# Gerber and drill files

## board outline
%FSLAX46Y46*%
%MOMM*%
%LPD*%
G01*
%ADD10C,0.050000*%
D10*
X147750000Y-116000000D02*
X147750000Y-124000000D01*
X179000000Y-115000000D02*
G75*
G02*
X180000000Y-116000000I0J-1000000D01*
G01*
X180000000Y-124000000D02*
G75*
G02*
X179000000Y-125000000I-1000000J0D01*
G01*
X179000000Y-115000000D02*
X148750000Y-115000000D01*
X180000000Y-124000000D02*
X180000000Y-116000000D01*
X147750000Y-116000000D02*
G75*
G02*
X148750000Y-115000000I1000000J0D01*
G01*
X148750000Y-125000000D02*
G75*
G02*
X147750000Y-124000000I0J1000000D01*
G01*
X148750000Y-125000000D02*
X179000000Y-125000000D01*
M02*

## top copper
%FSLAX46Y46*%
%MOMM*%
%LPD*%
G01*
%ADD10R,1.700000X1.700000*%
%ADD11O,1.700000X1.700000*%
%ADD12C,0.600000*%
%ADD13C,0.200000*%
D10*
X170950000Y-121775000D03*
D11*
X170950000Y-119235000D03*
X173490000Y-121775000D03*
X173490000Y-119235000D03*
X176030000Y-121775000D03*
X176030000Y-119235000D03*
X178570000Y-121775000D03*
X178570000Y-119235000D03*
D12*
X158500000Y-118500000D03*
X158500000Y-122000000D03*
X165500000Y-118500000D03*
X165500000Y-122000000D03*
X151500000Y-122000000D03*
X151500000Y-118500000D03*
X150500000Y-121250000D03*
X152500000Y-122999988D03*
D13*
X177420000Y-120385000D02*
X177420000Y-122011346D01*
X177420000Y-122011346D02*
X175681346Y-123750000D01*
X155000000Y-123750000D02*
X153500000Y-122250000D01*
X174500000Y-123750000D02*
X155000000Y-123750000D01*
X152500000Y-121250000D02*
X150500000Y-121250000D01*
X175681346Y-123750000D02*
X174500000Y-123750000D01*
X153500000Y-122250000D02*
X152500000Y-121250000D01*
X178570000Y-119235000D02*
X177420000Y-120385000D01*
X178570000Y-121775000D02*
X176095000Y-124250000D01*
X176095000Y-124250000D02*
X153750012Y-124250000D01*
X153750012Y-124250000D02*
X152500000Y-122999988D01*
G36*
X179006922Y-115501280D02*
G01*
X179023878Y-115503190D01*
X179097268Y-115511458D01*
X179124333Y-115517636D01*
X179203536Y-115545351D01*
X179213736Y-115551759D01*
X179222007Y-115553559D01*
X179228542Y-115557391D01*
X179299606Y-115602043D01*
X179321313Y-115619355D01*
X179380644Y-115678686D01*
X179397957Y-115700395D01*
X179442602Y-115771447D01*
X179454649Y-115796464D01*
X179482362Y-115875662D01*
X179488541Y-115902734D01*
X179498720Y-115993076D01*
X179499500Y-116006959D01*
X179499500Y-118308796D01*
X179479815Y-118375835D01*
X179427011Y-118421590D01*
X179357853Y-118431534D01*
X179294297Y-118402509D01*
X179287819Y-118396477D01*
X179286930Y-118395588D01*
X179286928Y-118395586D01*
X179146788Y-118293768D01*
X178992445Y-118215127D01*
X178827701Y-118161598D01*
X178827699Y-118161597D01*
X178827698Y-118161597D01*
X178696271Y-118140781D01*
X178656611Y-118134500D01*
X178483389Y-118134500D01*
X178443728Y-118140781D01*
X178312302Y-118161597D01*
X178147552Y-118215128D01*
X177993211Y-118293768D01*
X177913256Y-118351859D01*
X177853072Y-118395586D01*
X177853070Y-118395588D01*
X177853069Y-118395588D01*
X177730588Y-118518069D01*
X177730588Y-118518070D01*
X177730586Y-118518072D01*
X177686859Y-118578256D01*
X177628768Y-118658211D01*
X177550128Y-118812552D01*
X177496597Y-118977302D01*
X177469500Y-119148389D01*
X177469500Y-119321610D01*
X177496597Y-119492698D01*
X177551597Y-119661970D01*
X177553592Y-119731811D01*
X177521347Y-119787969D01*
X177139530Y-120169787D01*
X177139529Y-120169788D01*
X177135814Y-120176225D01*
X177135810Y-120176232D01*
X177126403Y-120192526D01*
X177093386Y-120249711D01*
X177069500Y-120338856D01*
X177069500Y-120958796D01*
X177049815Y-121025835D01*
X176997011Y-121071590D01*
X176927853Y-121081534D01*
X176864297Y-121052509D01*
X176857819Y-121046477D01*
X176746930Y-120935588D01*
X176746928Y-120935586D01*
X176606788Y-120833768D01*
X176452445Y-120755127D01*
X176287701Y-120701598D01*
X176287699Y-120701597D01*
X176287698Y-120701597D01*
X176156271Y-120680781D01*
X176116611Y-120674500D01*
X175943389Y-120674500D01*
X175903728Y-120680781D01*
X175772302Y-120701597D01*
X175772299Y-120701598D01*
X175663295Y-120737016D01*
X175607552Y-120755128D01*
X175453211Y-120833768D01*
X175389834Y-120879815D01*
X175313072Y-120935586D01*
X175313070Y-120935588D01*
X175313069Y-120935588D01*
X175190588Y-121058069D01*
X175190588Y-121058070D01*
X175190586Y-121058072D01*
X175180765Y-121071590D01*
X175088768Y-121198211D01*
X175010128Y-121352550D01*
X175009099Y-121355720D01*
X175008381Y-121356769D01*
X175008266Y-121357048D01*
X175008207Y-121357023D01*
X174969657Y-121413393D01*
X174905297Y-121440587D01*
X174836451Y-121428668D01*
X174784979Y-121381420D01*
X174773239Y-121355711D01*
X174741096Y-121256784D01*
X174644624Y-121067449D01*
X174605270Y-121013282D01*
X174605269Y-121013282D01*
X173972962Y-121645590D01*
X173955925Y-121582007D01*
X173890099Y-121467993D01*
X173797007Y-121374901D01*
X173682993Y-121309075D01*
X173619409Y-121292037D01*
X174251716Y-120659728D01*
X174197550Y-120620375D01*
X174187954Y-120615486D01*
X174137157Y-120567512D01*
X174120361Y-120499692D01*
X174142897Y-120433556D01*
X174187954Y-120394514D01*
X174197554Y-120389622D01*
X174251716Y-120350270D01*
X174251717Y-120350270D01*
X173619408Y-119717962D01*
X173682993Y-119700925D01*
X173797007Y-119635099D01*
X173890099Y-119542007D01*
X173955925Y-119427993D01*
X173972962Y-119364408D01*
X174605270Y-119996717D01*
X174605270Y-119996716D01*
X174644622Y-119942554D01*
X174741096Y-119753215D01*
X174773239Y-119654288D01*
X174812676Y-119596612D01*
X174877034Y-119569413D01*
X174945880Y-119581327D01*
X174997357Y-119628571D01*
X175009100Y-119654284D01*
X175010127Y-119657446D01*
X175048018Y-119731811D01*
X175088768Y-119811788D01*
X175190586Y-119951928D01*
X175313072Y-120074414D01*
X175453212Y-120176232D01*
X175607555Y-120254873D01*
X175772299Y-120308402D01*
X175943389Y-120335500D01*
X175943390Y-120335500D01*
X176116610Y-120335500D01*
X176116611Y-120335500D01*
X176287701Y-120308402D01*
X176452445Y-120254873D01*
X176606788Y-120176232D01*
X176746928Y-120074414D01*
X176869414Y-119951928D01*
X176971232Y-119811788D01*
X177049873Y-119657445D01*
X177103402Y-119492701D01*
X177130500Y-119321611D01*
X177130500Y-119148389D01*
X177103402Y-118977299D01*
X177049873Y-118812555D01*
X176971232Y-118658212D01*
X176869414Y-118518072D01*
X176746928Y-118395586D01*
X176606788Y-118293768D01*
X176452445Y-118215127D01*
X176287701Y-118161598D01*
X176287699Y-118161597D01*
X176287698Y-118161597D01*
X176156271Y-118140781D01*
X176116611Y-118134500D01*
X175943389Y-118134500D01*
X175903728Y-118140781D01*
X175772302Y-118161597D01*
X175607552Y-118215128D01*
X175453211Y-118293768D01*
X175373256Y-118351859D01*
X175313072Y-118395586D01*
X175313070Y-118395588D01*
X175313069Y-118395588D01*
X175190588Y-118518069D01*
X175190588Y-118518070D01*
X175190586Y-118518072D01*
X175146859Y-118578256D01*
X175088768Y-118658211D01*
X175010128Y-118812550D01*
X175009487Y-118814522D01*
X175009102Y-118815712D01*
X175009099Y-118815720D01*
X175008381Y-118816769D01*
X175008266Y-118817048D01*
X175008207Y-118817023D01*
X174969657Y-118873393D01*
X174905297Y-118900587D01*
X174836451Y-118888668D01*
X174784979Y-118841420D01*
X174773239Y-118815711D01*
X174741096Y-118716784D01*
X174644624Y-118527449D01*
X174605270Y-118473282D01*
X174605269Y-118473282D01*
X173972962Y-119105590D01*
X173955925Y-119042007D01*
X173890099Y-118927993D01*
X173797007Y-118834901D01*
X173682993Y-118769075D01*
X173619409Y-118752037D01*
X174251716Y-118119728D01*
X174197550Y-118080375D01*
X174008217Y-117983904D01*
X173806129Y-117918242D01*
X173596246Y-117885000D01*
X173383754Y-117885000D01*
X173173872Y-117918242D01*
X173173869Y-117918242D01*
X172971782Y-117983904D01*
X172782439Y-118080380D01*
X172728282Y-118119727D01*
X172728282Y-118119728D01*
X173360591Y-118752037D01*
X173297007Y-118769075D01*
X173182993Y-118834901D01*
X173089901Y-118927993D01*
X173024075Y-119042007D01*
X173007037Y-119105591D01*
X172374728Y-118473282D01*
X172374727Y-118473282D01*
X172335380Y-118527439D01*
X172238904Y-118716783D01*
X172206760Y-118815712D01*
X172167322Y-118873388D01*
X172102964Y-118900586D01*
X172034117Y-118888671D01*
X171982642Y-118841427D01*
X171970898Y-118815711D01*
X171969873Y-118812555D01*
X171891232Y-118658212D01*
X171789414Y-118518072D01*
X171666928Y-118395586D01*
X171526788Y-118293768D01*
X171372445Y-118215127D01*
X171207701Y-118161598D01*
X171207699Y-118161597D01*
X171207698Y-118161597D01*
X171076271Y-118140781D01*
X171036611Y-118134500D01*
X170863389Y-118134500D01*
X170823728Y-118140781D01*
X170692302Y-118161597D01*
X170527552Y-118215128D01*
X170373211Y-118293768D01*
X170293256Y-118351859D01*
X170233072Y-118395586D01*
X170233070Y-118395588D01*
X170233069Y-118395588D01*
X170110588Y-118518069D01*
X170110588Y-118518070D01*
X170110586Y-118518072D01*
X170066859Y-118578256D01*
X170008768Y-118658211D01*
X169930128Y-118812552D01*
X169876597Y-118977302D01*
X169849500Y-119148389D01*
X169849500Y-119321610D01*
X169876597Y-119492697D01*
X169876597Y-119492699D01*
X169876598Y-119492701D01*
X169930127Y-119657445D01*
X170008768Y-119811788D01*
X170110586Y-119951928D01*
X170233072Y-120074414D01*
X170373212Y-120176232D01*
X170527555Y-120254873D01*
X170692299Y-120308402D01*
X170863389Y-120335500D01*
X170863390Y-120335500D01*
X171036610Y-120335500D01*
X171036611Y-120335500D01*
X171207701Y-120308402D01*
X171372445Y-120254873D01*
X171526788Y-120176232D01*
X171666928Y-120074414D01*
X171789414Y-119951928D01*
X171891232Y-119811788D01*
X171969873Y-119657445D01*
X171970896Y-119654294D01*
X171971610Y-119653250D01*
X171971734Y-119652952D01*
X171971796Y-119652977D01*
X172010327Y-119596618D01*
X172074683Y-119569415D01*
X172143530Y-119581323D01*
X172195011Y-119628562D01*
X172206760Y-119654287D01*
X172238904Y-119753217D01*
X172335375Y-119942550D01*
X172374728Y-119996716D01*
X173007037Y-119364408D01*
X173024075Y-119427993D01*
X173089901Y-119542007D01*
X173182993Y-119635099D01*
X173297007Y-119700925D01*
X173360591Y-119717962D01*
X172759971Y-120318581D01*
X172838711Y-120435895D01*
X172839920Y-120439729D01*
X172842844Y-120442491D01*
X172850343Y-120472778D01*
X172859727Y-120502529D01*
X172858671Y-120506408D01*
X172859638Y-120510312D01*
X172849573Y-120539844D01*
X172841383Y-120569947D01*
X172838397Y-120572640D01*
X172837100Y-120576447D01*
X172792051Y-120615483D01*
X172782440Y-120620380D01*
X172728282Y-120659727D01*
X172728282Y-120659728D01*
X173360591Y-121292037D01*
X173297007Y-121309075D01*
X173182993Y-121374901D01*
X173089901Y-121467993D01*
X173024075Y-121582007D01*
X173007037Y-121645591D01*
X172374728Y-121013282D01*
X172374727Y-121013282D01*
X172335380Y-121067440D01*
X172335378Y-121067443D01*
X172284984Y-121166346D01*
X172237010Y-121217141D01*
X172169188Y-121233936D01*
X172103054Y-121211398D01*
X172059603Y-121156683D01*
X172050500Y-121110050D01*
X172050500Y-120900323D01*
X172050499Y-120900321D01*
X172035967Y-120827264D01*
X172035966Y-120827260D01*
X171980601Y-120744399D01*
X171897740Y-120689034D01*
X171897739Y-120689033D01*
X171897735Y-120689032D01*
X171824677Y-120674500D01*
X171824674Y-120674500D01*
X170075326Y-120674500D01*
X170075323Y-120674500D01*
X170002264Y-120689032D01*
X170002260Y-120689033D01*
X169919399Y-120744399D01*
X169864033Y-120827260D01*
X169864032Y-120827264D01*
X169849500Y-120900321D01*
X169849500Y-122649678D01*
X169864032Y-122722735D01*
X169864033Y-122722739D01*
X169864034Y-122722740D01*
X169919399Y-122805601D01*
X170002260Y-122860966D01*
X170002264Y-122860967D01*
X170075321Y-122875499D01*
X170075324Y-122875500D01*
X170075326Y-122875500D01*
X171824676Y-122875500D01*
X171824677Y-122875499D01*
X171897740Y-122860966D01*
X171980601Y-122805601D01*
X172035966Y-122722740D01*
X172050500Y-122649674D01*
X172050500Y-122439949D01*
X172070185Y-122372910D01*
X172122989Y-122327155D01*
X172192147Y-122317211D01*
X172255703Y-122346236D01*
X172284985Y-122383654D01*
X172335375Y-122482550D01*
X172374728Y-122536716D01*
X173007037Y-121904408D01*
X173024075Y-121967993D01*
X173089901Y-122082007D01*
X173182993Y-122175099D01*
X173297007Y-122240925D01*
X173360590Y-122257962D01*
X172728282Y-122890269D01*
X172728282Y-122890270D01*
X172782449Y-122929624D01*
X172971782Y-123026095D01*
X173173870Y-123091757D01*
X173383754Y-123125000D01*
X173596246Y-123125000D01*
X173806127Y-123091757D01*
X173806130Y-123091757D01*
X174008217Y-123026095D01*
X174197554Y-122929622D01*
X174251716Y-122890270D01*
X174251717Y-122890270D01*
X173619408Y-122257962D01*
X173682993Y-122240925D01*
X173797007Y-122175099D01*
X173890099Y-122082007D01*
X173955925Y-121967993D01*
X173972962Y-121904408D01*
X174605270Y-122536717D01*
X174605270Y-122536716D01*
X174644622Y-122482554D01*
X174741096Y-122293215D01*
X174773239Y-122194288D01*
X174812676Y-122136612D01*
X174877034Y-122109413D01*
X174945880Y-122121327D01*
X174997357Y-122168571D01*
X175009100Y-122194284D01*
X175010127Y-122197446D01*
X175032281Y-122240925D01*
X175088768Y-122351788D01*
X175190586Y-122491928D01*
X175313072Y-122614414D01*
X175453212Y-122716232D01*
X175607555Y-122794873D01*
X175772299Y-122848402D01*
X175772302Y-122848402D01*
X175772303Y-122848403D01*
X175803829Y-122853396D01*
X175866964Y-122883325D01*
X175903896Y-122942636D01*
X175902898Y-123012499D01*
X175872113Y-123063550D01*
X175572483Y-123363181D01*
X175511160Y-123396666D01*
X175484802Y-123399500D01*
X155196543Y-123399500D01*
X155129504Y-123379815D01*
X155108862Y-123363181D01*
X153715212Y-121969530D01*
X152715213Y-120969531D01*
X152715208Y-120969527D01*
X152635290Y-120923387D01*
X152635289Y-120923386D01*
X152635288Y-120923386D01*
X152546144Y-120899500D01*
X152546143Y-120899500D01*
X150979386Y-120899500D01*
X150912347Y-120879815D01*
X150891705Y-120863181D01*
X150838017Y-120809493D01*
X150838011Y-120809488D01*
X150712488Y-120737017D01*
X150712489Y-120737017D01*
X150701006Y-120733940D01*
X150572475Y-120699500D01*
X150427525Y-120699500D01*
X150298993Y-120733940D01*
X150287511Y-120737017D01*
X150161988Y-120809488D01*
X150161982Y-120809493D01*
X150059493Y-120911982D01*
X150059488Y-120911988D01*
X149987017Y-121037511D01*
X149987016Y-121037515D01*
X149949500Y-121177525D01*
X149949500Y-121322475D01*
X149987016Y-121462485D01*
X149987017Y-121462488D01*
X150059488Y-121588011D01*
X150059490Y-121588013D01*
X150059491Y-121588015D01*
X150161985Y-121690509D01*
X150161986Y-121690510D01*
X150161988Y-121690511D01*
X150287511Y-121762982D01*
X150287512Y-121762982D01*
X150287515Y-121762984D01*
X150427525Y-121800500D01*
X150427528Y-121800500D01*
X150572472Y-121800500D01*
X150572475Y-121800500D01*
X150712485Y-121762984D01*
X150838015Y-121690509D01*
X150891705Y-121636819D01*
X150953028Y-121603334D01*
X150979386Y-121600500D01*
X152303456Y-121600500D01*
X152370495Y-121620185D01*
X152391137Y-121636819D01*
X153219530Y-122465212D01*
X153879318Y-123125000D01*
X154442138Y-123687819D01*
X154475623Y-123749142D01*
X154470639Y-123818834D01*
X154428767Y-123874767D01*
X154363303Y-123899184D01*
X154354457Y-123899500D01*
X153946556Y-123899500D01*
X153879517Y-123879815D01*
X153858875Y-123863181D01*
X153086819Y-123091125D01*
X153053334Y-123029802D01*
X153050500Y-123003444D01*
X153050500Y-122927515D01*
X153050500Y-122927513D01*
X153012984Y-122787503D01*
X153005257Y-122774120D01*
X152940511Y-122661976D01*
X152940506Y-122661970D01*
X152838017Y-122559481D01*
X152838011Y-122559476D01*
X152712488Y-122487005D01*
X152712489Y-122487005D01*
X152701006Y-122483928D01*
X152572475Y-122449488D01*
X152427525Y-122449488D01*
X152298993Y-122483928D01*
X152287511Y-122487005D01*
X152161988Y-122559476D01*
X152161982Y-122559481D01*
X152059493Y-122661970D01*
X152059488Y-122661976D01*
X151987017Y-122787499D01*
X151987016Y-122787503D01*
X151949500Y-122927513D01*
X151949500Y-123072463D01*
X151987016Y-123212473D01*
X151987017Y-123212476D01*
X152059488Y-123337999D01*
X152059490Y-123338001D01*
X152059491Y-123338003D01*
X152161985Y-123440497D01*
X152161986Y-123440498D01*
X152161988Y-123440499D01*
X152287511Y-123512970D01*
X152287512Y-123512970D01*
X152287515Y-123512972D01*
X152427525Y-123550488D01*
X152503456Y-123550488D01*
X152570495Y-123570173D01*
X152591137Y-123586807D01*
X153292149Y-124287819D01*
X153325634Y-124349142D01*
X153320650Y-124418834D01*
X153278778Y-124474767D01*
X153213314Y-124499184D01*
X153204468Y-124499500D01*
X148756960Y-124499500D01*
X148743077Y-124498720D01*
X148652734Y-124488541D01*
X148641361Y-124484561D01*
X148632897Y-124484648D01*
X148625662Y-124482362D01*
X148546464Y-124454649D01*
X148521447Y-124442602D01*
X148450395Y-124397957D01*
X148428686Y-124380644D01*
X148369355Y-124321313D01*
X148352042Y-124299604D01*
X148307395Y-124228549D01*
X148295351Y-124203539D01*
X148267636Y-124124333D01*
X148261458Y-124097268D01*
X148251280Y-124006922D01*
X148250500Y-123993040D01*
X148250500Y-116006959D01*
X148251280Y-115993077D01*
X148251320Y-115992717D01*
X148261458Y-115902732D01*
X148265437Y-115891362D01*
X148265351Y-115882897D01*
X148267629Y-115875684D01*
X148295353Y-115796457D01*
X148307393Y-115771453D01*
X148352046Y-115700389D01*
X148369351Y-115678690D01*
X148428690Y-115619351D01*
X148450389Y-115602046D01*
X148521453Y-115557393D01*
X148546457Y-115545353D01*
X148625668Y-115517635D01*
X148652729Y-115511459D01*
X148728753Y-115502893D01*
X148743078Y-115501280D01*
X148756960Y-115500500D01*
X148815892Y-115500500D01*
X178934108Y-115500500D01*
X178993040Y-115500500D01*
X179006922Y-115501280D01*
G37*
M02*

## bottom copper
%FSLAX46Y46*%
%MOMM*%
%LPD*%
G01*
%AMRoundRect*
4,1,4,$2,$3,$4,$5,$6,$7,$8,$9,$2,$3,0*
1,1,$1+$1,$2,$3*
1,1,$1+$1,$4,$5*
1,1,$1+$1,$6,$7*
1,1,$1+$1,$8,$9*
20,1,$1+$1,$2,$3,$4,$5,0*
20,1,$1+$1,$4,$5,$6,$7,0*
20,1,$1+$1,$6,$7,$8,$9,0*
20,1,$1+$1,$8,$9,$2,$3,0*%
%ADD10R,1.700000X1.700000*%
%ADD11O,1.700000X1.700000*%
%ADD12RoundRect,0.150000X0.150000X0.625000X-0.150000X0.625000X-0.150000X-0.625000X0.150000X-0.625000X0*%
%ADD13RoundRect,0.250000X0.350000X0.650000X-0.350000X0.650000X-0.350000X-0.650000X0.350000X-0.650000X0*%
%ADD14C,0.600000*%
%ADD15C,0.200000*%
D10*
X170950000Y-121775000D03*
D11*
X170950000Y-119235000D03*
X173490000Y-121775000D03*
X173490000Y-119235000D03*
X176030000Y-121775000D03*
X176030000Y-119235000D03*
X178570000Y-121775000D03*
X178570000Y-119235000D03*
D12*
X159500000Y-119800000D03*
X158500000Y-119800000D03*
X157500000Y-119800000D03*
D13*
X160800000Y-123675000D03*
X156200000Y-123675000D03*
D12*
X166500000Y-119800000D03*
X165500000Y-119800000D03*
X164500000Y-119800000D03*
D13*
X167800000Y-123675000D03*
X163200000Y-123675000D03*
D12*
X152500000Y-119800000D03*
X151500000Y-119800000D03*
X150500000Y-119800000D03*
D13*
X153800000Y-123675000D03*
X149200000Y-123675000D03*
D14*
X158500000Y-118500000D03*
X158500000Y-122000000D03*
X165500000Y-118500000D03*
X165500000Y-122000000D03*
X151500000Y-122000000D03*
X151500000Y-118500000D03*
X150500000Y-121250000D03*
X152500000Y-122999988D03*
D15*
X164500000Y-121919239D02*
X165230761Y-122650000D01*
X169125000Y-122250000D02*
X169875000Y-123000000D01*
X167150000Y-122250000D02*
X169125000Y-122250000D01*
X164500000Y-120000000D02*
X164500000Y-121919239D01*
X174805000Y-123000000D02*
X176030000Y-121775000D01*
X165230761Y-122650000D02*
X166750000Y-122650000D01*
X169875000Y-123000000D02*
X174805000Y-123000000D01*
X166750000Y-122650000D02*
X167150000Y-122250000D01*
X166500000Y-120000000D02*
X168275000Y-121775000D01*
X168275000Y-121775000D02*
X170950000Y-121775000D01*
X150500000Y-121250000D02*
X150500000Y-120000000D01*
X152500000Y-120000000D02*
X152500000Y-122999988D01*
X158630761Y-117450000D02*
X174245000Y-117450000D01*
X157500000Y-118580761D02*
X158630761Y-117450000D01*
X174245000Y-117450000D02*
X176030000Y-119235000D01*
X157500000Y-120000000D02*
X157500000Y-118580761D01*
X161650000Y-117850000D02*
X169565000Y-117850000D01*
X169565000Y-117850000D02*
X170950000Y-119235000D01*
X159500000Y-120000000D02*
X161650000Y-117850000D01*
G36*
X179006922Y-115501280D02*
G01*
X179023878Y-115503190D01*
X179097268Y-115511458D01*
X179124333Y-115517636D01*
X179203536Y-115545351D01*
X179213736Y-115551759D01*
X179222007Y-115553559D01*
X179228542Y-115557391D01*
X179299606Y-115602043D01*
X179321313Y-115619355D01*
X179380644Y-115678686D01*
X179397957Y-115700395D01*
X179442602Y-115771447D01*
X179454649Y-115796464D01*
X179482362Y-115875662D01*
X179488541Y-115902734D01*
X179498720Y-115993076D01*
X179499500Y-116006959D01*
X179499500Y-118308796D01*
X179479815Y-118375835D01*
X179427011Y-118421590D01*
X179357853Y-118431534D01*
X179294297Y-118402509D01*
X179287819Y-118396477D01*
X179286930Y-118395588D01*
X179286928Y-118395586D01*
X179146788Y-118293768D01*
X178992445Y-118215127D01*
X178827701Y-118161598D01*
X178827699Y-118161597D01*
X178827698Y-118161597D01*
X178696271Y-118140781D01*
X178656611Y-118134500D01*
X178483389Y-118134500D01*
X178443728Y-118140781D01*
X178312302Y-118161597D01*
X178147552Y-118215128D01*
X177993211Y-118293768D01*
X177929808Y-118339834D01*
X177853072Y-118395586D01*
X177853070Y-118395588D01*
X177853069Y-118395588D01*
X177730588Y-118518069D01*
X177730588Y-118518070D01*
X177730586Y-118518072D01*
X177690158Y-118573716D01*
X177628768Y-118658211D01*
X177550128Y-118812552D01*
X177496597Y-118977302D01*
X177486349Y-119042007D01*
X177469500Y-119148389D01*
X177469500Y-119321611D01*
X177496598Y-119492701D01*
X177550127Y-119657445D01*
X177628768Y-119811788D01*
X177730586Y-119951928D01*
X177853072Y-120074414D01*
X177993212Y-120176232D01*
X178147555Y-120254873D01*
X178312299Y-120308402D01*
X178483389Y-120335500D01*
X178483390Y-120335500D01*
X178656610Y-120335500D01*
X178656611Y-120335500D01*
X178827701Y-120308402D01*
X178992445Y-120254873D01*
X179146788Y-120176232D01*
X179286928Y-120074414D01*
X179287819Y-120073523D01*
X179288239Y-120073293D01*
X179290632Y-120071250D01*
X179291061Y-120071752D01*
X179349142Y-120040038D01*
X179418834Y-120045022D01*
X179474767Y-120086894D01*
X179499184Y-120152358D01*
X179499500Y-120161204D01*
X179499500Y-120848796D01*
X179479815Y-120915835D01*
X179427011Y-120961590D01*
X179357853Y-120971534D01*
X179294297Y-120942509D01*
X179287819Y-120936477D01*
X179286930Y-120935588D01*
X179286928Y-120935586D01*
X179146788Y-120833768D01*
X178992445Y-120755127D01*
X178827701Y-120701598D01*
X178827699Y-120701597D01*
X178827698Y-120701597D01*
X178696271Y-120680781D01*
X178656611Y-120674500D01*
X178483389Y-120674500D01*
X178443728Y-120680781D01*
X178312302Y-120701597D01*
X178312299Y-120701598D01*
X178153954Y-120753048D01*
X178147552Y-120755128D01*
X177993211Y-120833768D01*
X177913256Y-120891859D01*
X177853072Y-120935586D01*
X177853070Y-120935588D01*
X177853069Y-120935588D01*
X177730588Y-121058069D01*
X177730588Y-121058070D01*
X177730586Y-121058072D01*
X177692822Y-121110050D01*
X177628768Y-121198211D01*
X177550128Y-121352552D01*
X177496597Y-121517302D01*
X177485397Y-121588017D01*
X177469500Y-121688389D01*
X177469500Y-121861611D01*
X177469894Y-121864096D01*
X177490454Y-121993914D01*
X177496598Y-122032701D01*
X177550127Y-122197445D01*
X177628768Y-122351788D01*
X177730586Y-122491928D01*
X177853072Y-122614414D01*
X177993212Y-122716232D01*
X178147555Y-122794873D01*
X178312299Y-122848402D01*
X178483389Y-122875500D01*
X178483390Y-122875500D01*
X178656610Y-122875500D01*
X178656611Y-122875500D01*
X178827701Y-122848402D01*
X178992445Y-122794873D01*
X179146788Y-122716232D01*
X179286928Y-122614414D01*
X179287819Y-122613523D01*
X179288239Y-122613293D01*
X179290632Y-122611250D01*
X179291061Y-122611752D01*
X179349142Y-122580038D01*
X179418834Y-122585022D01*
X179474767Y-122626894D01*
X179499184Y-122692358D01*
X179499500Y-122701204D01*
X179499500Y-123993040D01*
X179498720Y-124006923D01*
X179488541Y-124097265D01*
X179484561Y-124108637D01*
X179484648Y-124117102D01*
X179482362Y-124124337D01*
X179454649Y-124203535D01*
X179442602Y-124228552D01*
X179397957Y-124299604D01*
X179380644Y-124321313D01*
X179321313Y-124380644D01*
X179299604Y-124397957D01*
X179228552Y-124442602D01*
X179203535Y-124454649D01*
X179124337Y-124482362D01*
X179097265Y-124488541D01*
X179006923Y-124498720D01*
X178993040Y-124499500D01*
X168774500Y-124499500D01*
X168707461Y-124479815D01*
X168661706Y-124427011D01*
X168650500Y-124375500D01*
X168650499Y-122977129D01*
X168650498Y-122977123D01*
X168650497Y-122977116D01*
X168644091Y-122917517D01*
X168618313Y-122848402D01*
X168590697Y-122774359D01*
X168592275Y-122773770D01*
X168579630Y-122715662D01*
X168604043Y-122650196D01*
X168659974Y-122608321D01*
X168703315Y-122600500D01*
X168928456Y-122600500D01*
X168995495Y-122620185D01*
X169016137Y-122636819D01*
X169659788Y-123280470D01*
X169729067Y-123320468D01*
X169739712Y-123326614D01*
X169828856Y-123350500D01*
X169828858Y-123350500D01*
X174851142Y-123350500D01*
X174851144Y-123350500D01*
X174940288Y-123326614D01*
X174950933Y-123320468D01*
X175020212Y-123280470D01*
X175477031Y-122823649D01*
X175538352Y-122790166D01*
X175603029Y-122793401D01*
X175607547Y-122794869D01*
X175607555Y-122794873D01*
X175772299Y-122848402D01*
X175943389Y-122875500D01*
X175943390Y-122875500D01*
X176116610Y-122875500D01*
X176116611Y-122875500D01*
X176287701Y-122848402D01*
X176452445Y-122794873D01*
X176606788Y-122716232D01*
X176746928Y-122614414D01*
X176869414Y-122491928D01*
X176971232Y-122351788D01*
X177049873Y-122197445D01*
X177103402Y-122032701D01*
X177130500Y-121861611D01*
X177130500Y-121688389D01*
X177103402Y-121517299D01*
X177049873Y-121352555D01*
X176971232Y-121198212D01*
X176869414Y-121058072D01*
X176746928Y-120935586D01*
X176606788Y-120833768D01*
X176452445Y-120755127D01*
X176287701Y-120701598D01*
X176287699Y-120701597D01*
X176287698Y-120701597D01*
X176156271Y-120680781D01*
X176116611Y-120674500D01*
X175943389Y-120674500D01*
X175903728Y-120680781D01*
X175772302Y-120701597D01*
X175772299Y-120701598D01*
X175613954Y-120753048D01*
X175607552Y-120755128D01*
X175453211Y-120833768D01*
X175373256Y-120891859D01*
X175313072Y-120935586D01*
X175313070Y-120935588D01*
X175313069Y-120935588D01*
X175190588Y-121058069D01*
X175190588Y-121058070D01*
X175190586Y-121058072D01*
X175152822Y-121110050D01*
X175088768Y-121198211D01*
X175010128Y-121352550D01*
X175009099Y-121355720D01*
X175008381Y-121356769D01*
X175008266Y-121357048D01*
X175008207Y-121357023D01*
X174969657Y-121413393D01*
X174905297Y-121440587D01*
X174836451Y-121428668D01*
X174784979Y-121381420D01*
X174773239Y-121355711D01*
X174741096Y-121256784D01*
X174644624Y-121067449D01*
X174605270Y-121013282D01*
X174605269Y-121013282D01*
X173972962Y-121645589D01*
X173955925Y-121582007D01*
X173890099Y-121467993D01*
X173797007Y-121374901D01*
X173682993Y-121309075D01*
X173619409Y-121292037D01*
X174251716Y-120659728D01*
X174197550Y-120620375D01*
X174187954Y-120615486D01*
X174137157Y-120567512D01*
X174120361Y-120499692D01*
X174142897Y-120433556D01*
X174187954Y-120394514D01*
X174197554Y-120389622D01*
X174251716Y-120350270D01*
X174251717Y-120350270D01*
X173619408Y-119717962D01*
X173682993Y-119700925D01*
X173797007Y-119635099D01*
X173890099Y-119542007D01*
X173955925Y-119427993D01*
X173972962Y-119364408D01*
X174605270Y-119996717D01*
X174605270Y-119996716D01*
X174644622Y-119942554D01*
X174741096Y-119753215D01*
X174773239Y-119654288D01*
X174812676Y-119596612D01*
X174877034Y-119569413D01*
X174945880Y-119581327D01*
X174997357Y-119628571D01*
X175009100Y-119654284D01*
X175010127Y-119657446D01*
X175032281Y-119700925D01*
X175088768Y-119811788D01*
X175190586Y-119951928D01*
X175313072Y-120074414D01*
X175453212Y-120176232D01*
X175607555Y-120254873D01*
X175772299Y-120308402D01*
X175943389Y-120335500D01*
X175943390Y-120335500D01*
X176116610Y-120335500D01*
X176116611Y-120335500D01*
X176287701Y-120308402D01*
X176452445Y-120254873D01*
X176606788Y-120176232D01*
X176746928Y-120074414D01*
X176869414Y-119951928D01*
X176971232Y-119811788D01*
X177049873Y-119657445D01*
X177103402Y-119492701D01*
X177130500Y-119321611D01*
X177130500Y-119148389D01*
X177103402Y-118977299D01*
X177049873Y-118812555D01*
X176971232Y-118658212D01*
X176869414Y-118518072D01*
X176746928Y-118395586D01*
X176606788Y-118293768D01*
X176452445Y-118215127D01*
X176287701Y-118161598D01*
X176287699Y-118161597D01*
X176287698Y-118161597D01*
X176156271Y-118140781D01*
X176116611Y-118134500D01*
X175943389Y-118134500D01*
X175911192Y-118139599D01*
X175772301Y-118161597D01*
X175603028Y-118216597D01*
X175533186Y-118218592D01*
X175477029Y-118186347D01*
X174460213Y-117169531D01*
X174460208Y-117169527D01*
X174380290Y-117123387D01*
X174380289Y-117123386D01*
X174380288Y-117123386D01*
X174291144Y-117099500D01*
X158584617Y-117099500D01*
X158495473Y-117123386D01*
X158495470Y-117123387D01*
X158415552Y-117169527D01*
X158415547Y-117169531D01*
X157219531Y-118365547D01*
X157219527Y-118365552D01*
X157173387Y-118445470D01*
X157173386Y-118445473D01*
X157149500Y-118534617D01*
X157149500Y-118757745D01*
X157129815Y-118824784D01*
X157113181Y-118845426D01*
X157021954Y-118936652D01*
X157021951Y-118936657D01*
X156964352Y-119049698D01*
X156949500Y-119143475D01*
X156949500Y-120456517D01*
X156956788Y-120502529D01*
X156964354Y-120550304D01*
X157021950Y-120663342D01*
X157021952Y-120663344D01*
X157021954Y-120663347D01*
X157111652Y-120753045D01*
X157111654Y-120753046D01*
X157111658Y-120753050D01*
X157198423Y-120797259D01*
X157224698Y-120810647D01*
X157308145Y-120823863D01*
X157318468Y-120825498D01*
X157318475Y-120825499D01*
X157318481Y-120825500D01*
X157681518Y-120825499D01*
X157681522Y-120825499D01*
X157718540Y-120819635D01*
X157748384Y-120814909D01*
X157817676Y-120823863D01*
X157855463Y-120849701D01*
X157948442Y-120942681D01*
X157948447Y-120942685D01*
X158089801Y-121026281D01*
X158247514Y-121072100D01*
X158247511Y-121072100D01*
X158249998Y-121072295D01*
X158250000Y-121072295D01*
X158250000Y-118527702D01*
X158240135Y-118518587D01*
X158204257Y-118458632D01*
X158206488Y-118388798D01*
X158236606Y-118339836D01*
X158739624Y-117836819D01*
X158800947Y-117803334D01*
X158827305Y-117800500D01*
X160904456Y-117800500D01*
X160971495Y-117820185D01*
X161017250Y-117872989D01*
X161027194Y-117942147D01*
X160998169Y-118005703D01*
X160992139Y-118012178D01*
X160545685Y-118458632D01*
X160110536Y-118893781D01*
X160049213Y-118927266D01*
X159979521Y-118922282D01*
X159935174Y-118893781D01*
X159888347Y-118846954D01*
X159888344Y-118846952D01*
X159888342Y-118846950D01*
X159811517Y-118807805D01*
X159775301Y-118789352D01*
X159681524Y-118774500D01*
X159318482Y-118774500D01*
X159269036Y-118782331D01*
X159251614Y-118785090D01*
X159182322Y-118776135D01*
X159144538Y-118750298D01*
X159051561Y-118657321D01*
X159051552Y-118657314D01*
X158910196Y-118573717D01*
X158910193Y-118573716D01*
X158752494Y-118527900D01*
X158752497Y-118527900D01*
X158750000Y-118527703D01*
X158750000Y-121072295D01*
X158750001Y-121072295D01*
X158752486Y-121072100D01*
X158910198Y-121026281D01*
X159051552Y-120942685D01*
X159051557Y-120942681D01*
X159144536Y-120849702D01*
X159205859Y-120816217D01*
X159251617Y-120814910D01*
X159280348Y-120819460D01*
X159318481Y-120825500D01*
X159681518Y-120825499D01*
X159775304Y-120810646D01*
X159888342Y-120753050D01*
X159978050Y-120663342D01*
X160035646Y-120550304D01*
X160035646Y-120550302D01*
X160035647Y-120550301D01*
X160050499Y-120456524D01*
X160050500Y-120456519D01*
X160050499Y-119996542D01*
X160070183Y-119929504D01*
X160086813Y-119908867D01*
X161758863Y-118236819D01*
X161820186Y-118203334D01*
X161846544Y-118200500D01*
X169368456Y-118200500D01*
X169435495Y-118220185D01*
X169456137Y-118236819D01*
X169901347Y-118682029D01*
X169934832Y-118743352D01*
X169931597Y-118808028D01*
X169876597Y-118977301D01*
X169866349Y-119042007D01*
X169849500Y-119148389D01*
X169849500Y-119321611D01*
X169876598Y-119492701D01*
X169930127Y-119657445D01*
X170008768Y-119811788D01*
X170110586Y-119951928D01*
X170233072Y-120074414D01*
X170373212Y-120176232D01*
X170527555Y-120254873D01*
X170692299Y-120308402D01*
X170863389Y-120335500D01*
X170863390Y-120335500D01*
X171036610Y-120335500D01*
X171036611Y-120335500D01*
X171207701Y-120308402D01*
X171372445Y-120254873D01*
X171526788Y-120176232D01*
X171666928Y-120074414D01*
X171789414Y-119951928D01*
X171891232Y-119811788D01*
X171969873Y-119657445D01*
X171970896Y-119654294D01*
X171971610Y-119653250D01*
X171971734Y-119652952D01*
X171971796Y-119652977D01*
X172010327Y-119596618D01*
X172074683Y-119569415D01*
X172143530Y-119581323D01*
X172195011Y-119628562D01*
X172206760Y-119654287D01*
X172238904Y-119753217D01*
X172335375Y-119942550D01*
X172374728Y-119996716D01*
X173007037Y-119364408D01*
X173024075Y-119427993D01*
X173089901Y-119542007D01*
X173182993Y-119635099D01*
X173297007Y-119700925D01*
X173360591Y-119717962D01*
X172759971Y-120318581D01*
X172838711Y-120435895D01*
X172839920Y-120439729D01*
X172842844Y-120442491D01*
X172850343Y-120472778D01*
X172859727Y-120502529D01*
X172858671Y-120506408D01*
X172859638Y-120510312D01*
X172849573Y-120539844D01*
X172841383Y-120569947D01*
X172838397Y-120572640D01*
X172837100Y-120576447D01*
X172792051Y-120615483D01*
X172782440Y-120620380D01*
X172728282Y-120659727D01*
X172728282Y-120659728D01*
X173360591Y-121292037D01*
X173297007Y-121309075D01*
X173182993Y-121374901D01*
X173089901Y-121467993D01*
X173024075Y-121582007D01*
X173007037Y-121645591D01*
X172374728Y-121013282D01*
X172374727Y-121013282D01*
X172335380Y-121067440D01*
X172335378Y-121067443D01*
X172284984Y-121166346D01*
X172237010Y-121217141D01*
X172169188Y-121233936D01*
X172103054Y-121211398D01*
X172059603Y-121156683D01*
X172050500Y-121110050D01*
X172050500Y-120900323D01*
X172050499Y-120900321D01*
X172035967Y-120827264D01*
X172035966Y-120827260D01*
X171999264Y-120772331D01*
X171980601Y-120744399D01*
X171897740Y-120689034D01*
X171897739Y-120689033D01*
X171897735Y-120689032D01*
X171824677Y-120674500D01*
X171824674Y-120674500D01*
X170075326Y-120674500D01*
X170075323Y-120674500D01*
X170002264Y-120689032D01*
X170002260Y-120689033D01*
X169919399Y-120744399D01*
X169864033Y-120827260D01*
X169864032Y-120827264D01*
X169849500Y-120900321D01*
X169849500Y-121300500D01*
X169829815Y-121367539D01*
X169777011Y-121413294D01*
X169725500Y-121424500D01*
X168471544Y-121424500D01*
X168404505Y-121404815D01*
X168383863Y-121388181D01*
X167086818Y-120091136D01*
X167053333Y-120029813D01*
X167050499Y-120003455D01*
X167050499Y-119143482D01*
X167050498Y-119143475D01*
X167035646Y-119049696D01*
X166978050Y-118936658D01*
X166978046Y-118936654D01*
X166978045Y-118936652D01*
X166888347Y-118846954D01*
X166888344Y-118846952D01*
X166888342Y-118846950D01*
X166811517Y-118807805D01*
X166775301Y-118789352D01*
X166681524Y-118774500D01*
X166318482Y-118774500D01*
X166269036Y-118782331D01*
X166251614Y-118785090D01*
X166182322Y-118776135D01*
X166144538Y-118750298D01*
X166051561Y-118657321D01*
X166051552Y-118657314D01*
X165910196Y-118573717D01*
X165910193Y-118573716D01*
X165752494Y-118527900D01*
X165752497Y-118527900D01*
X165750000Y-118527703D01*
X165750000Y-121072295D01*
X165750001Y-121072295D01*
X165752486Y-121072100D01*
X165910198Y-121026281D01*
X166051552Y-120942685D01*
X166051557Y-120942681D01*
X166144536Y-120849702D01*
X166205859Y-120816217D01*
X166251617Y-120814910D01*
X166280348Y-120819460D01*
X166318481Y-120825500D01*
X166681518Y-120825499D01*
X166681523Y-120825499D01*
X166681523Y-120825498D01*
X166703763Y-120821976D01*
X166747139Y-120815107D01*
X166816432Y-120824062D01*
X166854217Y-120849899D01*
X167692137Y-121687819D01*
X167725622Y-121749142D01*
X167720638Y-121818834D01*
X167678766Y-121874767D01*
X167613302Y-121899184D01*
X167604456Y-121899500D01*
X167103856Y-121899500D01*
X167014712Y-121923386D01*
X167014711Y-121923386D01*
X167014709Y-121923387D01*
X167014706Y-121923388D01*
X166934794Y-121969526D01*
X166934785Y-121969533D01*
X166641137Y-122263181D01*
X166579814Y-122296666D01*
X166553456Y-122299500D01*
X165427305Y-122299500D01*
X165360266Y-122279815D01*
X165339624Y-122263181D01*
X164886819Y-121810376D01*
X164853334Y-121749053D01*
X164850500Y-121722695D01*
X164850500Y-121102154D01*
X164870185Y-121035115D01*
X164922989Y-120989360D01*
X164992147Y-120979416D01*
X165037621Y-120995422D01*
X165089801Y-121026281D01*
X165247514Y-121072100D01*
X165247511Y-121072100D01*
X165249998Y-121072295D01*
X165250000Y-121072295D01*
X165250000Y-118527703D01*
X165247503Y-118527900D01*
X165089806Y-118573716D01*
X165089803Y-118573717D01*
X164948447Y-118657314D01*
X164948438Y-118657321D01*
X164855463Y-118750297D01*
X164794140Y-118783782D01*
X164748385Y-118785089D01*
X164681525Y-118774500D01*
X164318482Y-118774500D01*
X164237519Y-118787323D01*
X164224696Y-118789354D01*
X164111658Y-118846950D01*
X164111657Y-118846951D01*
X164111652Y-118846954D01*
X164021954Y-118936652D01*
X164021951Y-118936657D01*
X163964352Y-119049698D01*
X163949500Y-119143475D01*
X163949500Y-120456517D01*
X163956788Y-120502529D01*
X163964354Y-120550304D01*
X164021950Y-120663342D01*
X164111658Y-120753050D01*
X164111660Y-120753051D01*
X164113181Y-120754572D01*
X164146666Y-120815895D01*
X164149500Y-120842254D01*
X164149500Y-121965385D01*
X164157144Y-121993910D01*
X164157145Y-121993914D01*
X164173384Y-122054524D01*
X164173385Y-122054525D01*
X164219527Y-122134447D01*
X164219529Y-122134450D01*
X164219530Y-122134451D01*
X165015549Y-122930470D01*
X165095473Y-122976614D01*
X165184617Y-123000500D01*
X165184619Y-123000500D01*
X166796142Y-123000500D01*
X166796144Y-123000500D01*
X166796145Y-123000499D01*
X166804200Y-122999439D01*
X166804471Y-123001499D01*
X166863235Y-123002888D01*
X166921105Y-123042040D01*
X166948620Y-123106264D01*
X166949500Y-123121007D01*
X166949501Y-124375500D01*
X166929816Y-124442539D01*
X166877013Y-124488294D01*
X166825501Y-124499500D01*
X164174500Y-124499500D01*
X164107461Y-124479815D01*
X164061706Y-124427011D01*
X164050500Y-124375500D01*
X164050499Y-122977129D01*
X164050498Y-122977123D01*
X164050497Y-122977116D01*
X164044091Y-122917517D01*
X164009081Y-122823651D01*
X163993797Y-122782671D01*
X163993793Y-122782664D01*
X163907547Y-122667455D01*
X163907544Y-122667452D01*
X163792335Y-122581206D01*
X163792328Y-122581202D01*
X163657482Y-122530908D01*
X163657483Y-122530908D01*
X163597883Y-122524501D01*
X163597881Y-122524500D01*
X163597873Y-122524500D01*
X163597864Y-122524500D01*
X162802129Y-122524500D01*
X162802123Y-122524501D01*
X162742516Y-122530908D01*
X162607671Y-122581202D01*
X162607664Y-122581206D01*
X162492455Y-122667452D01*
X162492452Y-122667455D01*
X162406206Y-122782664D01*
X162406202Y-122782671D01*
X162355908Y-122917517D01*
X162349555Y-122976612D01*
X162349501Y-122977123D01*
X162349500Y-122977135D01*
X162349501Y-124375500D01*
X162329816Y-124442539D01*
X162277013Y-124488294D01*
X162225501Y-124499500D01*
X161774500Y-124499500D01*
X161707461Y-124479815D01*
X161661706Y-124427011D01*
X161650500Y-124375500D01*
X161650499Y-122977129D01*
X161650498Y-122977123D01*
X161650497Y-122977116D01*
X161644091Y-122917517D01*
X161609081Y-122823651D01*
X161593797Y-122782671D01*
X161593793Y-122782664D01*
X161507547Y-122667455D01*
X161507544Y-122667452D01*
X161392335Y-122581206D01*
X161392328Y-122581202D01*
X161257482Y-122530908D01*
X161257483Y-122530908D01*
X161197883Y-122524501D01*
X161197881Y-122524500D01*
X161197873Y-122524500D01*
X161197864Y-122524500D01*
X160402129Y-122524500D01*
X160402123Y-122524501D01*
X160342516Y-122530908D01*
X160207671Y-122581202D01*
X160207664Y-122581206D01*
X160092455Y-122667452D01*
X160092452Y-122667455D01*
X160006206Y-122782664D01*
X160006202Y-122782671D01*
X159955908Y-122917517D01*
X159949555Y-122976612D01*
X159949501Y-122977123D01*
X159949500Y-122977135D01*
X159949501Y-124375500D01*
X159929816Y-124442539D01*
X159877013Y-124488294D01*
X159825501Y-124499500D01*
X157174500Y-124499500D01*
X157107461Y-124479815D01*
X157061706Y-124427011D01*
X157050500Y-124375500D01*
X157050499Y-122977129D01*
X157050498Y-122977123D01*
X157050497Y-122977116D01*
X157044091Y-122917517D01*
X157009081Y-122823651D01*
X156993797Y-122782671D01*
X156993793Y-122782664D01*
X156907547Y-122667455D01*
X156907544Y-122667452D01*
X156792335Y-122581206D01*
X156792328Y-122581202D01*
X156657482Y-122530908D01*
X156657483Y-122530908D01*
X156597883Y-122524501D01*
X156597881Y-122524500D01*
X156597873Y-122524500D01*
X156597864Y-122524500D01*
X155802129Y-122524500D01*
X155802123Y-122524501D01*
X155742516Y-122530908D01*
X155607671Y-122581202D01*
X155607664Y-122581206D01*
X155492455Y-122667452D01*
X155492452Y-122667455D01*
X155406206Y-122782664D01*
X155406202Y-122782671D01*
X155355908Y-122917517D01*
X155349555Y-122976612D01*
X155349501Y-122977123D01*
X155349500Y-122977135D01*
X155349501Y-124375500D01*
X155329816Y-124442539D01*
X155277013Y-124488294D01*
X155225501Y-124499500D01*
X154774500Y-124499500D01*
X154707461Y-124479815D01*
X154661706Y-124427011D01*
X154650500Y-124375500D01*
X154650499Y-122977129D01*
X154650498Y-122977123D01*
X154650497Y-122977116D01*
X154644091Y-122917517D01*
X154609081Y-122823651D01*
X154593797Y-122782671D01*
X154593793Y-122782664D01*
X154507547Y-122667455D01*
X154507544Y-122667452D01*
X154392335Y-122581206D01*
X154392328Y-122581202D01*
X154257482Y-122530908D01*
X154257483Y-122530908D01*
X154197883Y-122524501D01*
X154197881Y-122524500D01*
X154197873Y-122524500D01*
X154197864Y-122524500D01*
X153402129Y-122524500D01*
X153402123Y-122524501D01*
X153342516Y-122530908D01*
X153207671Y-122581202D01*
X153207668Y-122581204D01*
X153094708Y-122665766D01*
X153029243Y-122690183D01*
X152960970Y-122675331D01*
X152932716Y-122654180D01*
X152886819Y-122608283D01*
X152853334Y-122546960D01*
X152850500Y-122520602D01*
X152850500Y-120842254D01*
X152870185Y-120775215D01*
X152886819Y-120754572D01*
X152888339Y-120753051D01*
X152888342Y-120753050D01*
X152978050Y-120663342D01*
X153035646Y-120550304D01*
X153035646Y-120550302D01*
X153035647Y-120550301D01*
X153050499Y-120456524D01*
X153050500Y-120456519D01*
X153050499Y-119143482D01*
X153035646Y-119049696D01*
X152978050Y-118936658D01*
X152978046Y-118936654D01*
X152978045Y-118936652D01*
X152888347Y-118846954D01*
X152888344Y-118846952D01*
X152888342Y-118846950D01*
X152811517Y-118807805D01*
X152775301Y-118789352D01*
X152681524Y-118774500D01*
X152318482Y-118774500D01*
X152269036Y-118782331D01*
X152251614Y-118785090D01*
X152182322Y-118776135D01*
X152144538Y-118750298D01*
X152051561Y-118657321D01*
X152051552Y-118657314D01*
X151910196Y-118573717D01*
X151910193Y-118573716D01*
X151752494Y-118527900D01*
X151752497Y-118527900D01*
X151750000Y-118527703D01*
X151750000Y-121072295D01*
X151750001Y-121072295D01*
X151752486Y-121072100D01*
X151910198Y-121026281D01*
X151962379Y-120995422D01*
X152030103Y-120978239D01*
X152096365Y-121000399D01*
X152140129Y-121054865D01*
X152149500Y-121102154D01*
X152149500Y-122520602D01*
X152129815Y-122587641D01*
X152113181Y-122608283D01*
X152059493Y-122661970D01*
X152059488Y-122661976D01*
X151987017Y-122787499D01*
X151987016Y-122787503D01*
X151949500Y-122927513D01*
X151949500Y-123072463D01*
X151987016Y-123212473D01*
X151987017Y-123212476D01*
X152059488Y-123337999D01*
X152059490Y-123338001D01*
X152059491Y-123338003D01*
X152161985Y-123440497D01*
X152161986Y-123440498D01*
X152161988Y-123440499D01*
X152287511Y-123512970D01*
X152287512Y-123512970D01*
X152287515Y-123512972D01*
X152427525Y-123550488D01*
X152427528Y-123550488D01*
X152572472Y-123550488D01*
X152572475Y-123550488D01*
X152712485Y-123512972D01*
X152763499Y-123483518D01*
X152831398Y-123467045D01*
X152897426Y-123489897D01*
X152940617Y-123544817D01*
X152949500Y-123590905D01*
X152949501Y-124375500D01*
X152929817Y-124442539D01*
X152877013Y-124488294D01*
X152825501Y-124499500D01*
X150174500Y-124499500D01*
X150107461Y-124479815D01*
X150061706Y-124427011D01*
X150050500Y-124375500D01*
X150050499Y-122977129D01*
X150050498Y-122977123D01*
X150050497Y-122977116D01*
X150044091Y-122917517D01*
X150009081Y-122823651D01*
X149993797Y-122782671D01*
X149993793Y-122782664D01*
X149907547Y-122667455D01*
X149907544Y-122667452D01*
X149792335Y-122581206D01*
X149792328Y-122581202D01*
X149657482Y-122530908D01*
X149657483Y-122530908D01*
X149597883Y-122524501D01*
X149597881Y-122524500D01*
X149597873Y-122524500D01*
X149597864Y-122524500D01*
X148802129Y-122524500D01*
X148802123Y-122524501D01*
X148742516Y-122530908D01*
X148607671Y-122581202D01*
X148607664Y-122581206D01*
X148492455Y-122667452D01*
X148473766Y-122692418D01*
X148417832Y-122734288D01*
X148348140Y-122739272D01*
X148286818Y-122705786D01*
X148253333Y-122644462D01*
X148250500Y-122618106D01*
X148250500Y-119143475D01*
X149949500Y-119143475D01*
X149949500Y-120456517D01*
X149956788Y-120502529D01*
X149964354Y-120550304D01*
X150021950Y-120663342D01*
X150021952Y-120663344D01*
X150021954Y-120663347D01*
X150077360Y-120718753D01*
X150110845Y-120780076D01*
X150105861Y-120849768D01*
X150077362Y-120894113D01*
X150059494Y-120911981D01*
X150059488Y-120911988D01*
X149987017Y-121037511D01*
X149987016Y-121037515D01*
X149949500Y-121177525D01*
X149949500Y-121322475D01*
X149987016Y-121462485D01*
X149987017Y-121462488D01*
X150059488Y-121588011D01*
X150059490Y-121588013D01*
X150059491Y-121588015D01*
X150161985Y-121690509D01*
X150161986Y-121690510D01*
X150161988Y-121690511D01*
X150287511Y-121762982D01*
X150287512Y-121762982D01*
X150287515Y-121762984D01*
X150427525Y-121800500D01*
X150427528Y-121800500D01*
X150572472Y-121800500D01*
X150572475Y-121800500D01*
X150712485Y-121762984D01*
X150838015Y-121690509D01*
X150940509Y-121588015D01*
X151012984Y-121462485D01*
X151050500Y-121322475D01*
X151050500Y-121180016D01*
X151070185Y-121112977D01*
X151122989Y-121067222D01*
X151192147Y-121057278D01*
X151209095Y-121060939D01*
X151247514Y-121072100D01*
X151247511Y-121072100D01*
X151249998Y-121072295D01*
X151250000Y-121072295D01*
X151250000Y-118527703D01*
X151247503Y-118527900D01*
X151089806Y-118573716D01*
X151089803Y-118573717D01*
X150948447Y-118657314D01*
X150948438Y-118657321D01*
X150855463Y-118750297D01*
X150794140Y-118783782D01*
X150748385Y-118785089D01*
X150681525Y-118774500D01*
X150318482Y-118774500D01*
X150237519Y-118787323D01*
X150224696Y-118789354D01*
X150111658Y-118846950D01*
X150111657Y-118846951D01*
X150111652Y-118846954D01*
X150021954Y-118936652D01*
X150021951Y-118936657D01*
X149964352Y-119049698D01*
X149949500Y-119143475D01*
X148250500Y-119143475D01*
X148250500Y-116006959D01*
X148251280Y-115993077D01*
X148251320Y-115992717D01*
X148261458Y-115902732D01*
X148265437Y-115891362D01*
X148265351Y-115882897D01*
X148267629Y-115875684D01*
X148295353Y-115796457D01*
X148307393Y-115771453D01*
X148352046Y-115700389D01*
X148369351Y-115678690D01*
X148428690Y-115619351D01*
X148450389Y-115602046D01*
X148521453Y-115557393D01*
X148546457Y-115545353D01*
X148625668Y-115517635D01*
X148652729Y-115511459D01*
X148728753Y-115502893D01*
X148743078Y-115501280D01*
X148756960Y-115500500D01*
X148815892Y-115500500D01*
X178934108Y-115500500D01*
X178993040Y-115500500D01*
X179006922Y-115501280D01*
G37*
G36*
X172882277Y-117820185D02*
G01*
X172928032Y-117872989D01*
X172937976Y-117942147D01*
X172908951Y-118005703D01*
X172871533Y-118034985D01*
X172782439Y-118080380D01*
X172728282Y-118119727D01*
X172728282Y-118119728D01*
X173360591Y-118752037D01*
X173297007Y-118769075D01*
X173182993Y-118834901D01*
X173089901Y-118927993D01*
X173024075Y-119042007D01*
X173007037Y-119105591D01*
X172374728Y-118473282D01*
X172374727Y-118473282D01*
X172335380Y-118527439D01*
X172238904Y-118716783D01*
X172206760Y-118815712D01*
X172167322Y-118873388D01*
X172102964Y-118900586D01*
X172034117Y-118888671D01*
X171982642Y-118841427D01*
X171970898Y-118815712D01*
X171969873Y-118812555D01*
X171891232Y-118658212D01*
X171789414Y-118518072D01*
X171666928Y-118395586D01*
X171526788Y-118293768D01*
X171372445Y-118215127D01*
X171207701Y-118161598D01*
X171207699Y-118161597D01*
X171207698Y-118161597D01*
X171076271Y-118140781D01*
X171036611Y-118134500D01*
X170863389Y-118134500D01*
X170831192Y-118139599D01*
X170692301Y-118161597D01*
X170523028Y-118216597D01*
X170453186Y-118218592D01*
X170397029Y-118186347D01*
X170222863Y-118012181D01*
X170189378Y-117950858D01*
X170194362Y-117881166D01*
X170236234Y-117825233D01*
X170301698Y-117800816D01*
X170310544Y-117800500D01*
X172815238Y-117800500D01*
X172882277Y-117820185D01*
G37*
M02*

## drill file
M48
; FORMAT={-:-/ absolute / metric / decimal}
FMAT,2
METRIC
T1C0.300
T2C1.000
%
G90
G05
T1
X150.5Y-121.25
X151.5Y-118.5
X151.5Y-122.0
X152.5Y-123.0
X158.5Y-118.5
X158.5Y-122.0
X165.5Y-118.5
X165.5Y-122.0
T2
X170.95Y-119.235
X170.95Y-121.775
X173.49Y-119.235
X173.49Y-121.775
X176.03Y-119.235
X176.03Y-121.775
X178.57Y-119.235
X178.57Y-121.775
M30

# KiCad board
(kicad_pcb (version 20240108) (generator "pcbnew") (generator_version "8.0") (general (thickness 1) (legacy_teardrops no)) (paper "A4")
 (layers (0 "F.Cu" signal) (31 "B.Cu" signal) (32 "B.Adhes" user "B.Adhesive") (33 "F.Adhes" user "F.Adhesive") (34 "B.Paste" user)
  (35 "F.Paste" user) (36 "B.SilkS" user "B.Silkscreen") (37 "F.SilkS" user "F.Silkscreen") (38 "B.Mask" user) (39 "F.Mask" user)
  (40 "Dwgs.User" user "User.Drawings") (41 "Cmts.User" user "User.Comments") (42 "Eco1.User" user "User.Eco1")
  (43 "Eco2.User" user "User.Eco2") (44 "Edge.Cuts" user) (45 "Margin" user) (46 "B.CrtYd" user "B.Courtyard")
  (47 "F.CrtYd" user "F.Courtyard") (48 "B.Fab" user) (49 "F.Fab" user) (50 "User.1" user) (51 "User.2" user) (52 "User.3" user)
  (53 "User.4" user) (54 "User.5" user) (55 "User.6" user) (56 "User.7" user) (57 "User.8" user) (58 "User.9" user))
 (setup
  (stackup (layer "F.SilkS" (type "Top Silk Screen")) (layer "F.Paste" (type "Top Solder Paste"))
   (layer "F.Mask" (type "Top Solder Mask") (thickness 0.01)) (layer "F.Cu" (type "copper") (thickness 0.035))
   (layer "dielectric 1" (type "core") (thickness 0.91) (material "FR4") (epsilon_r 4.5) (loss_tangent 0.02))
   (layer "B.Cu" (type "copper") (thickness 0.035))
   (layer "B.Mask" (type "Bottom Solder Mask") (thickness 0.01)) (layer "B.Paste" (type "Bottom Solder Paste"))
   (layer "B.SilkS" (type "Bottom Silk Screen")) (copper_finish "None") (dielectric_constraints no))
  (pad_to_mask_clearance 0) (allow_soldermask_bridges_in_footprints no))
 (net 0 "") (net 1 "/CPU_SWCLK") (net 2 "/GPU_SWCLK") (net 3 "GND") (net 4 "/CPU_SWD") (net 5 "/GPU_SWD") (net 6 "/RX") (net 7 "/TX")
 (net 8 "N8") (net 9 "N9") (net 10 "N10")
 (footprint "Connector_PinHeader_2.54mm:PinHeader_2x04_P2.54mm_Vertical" (layer "F.Cu") (at 170.95 121.775 90)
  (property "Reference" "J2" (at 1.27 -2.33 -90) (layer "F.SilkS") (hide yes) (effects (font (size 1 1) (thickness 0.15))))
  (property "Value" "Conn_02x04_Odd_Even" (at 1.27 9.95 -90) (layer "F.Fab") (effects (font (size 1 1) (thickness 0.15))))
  (pad "1" thru_hole rect (at 0 0 90) (size 1.7 1.7) (drill 1) (layers "*.Cu" "*.Mask") (remove_unused_layers no) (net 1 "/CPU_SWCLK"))
  (pad "2" thru_hole oval (at 2.54 0 90) (size 1.7 1.7) (drill 1) (layers "*.Cu" "*.Mask") (remove_unused_layers no) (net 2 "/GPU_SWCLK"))
  (pad "3" thru_hole oval (at 0 2.54 90) (size 1.7 1.7) (drill 1) (layers "*.Cu" "*.Mask") (remove_unused_layers no) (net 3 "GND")
   (thermal_bridge_angle 45))
  (pad "4" thru_hole oval (at 2.54 2.54 90) (size 1.7 1.7) (drill 1) (layers "*.Cu" "*.Mask") (remove_unused_layers no) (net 3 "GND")
   (thermal_bridge_angle 45))
  (pad "5" thru_hole oval (at 0 5.08 90) (size 1.7 1.7) (drill 1) (layers "*.Cu" "*.Mask") (remove_unused_layers no) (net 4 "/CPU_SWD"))
  (pad "6" thru_hole oval (at 2.54 5.08 90) (size 1.7 1.7) (drill 1) (layers "*.Cu" "*.Mask") (remove_unused_layers no) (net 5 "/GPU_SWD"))
  (pad "7" thru_hole oval (at 0 7.62 90) (size 1.7 1.7) (drill 1) (layers "*.Cu" "*.Mask") (remove_unused_layers no) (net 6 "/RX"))
  (pad "8" thru_hole oval (at 2.54 7.62 90) (size 1.7 1.7) (drill 1) (layers "*.Cu" "*.Mask") (remove_unused_layers no) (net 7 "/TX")))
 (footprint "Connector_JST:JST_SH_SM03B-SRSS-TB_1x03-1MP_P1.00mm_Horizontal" (layer "B.Cu") (at 158.5 121.8 180)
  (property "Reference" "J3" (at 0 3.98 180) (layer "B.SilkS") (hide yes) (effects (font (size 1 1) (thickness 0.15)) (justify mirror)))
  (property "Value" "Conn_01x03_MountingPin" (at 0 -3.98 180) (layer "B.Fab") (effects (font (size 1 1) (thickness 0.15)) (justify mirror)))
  (pad "1" smd roundrect (at -1 2 180) (size 0.6 1.55) (layers "B.Cu" "B.Paste" "B.Mask") (roundrect_rratio 0.25) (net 2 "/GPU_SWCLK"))
  (pad "2" smd roundrect (at 0 2 180) (size 0.6 1.55) (layers "B.Cu" "B.Paste" "B.Mask") (roundrect_rratio 0.25) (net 3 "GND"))
  (pad "3" smd roundrect (at 1 2 180) (size 0.6 1.55) (layers "B.Cu" "B.Paste" "B.Mask") (roundrect_rratio 0.25) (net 5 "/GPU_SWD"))
  (pad "MP" smd roundrect (at -2.3 -1.875 180) (size 1.2 1.8) (layers "B.Cu" "B.Paste" "B.Mask") (roundrect_rratio 0.208333) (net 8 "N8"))
  (pad "MP" smd roundrect (at 2.3 -1.875 180) (size 1.2 1.8) (layers "B.Cu" "B.Paste" "B.Mask") (roundrect_rratio 0.208333) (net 8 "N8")))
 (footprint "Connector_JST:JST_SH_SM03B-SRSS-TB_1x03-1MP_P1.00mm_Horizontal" (layer "B.Cu") (at 165.5 121.8 180)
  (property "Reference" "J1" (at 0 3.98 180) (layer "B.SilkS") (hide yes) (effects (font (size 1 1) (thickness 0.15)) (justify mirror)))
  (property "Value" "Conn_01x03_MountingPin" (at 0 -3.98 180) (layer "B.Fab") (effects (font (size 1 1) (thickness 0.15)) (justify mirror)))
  (pad "1" smd roundrect (at -1 2 180) (size 0.6 1.55) (layers "B.Cu" "B.Paste" "B.Mask") (roundrect_rratio 0.25) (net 1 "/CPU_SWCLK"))
  (pad "2" smd roundrect (at 0 2 180) (size 0.6 1.55) (layers "B.Cu" "B.Paste" "B.Mask") (roundrect_rratio 0.25) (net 3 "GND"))
  (pad "3" smd roundrect (at 1 2 180) (size 0.6 1.55) (layers "B.Cu" "B.Paste" "B.Mask") (roundrect_rratio 0.25) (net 4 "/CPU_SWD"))
  (pad "MP" smd roundrect (at -2.3 -1.875 180) (size 1.2 1.8) (layers "B.Cu" "B.Paste" "B.Mask") (roundrect_rratio 0.208333) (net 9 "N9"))
  (pad "MP" smd roundrect (at 2.3 -1.875 180) (size 1.2 1.8) (layers "B.Cu" "B.Paste" "B.Mask") (roundrect_rratio 0.208333) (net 9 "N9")))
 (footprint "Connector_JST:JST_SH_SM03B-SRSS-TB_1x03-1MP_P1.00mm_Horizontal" (layer "B.Cu") (at 151.5 121.8 180)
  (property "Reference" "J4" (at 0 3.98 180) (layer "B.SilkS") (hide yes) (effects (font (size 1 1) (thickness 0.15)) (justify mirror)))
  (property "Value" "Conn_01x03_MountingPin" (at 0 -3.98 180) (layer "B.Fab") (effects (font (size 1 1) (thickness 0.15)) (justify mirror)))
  (pad "1" smd roundrect (at -1 2 180) (size 0.6 1.55) (layers "B.Cu" "B.Paste" "B.Mask") (roundrect_rratio 0.25) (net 6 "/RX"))
  (pad "2" smd roundrect (at 0 2 180) (size 0.6 1.55) (layers "B.Cu" "B.Paste" "B.Mask") (roundrect_rratio 0.25) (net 3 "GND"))
  (pad "3" smd roundrect (at 1 2 180) (size 0.6 1.55) (layers "B.Cu" "B.Paste" "B.Mask") (roundrect_rratio 0.25) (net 7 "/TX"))
  (pad "MP" smd roundrect (at -2.3 -1.875 180) (size 1.2 1.8) (layers "B.Cu" "B.Paste" "B.Mask") (roundrect_rratio 0.208333) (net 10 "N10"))
  (pad "MP" smd roundrect (at 2.3 -1.875 180) (size 1.2 1.8) (layers "B.Cu" "B.Paste" "B.Mask") (roundrect_rratio 0.208333) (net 10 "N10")))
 (gr_line (start 147.75 116) (end 147.75 124) (stroke (width 0.05) (type default)) (layer "Edge.Cuts"))
 (gr_arc (start 179 115) (mid 179.707107 115.292893) (end 180 116) (stroke (width 0.05) (type default)) (layer "Edge.Cuts"))
 (gr_arc (start 180 124) (mid 179.707107 124.707107) (end 179 125) (stroke (width 0.05) (type default)) (layer "Edge.Cuts"))
 (gr_line (start 179 115) (end 148.75 115) (stroke (width 0.05) (type default)) (layer "Edge.Cuts"))
 (gr_line (start 180 124) (end 180 116) (stroke (width 0.05) (type default)) (layer "Edge.Cuts"))
 (gr_arc (start 147.75 116) (mid 148.042893 115.292893) (end 148.75 115) (stroke (width 0.05) (type default)) (layer "Edge.Cuts"))
 (gr_arc (start 148.75 125) (mid 148.042893 124.707107) (end 147.75 124) (stroke (width 0.05) (type default)) (layer "Edge.Cuts"))
 (gr_line (start 148.75 125) (end 179 125) (stroke (width 0.05) (type default)) (layer "Edge.Cuts"))
 (via (at 158.5 118.5) (size 0.6) (drill 0.3) (layers "F.Cu" "B.Cu") (free yes) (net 3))
 (via (at 158.5 122) (size 0.6) (drill 0.3) (layers "F.Cu" "B.Cu") (free yes) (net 3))
 (via (at 165.5 118.5) (size 0.6) (drill 0.3) (layers "F.Cu" "B.Cu") (free yes) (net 3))
 (via (at 165.5 122) (size 0.6) (drill 0.3) (layers "F.Cu" "B.Cu") (free yes) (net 3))
 (via (at 151.5 122) (size 0.6) (drill 0.3) (layers "F.Cu" "B.Cu") (free yes) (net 3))
 (via (at 151.5 118.5) (size 0.6) (drill 0.3) (layers "F.Cu" "B.Cu") (free yes) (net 3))
 (segment (start 164.5 121.919239) (end 165.230761 122.65) (width 0.2) (layer "B.Cu") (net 4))
 (segment (start 169.125 122.25) (end 169.875 123) (width 0.2) (layer "B.Cu") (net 4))
 (segment (start 167.15 122.25) (end 169.125 122.25) (width 0.2) (layer "B.Cu") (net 4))
 (segment (start 164.5 120) (end 164.5 121.919239) (width 0.2) (layer "B.Cu") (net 4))
 (segment (start 174.805 123) (end 176.03 121.775) (width 0.2) (layer "B.Cu") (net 4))
 (segment (start 165.230761 122.65) (end 166.75 122.65) (width 0.2) (layer "B.Cu") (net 4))
 (segment (start 169.875 123) (end 174.805 123) (width 0.2) (layer "B.Cu") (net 4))
 (segment (start 166.75 122.65) (end 167.15 122.25) (width 0.2) (layer "B.Cu") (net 4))
 (segment (start 166.5 120) (end 168.275 121.775) (width 0.2) (layer "B.Cu") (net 1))
 (segment (start 168.275 121.775) (end 170.95 121.775) (width 0.2) (layer "B.Cu") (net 1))
 (segment (start 177.42 120.385) (end 177.42 122.011346) (width 0.2) (layer "F.Cu") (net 7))
 (segment (start 177.42 122.011346) (end 175.681346 123.75) (width 0.2) (layer "F.Cu") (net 7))
 (segment (start 155 123.75) (end 153.5 122.25) (width 0.2) (layer "F.Cu") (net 7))
 (segment (start 174.5 123.75) (end 155 123.75) (width 0.2) (layer "F.Cu") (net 7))
 (segment (start 152.5 121.25) (end 150.5 121.25) (width 0.2) (layer "F.Cu") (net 7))
 (segment (start 175.681346 123.75) (end 174.5 123.75) (width 0.2) (layer "F.Cu") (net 7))
 (segment (start 153.5 122.25) (end 152.5 121.25) (width 0.2) (layer "F.Cu") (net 7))
 (segment (start 178.57 119.235) (end 177.42 120.385) (width 0.2) (layer "F.Cu") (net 7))
 (via (at 150.5 121.25) (size 0.6) (drill 0.3) (layers "F.Cu" "B.Cu") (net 7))
 (segment (start 150.5 121.25) (end 150.5 120) (width 0.2) (layer "B.Cu") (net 7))
 (segment (start 178.57 121.775) (end 176.095 124.25) (width 0.2) (layer "F.Cu") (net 6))
 (segment (start 176.095 124.25) (end 153.750012 124.25) (width 0.2) (layer "F.Cu") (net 6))
 (segment (start 153.750012 124.25) (end 152.5 122.999988) (width 0.2) (layer "F.Cu") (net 6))
 (via (at 152.5 122.999988) (size 0.6) (drill 0.3) (layers "F.Cu" "B.Cu") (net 6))
 (segment (start 152.5 120) (end 152.5 122.999988) (width 0.2) (layer "B.Cu") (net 6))
 (segment (start 158.630761 117.45) (end 174.245 117.45) (width 0.2) (layer "B.Cu") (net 5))
 (segment (start 157.5 118.580761) (end 158.630761 117.45) (width 0.2) (layer "B.Cu") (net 5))
 (segment (start 174.245 117.45) (end 176.03 119.235) (width 0.2) (layer "B.Cu") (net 5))
 (segment (start 157.5 120) (end 157.5 118.580761) (width 0.2) (layer "B.Cu") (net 5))
 (segment (start 161.65 117.85) (end 169.565 117.85) (width 0.2) (layer "B.Cu") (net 2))
 (segment (start 169.565 117.85) (end 170.95 119.235) (width 0.2) (layer "B.Cu") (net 2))
 (segment (start 159.5 120) (end 161.65 117.85) (width 0.2) (layer "B.Cu") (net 2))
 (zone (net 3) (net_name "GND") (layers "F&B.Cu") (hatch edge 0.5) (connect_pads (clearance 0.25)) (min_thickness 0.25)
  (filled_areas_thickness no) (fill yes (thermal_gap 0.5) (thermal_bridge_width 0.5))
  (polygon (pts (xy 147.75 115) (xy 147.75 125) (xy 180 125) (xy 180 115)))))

